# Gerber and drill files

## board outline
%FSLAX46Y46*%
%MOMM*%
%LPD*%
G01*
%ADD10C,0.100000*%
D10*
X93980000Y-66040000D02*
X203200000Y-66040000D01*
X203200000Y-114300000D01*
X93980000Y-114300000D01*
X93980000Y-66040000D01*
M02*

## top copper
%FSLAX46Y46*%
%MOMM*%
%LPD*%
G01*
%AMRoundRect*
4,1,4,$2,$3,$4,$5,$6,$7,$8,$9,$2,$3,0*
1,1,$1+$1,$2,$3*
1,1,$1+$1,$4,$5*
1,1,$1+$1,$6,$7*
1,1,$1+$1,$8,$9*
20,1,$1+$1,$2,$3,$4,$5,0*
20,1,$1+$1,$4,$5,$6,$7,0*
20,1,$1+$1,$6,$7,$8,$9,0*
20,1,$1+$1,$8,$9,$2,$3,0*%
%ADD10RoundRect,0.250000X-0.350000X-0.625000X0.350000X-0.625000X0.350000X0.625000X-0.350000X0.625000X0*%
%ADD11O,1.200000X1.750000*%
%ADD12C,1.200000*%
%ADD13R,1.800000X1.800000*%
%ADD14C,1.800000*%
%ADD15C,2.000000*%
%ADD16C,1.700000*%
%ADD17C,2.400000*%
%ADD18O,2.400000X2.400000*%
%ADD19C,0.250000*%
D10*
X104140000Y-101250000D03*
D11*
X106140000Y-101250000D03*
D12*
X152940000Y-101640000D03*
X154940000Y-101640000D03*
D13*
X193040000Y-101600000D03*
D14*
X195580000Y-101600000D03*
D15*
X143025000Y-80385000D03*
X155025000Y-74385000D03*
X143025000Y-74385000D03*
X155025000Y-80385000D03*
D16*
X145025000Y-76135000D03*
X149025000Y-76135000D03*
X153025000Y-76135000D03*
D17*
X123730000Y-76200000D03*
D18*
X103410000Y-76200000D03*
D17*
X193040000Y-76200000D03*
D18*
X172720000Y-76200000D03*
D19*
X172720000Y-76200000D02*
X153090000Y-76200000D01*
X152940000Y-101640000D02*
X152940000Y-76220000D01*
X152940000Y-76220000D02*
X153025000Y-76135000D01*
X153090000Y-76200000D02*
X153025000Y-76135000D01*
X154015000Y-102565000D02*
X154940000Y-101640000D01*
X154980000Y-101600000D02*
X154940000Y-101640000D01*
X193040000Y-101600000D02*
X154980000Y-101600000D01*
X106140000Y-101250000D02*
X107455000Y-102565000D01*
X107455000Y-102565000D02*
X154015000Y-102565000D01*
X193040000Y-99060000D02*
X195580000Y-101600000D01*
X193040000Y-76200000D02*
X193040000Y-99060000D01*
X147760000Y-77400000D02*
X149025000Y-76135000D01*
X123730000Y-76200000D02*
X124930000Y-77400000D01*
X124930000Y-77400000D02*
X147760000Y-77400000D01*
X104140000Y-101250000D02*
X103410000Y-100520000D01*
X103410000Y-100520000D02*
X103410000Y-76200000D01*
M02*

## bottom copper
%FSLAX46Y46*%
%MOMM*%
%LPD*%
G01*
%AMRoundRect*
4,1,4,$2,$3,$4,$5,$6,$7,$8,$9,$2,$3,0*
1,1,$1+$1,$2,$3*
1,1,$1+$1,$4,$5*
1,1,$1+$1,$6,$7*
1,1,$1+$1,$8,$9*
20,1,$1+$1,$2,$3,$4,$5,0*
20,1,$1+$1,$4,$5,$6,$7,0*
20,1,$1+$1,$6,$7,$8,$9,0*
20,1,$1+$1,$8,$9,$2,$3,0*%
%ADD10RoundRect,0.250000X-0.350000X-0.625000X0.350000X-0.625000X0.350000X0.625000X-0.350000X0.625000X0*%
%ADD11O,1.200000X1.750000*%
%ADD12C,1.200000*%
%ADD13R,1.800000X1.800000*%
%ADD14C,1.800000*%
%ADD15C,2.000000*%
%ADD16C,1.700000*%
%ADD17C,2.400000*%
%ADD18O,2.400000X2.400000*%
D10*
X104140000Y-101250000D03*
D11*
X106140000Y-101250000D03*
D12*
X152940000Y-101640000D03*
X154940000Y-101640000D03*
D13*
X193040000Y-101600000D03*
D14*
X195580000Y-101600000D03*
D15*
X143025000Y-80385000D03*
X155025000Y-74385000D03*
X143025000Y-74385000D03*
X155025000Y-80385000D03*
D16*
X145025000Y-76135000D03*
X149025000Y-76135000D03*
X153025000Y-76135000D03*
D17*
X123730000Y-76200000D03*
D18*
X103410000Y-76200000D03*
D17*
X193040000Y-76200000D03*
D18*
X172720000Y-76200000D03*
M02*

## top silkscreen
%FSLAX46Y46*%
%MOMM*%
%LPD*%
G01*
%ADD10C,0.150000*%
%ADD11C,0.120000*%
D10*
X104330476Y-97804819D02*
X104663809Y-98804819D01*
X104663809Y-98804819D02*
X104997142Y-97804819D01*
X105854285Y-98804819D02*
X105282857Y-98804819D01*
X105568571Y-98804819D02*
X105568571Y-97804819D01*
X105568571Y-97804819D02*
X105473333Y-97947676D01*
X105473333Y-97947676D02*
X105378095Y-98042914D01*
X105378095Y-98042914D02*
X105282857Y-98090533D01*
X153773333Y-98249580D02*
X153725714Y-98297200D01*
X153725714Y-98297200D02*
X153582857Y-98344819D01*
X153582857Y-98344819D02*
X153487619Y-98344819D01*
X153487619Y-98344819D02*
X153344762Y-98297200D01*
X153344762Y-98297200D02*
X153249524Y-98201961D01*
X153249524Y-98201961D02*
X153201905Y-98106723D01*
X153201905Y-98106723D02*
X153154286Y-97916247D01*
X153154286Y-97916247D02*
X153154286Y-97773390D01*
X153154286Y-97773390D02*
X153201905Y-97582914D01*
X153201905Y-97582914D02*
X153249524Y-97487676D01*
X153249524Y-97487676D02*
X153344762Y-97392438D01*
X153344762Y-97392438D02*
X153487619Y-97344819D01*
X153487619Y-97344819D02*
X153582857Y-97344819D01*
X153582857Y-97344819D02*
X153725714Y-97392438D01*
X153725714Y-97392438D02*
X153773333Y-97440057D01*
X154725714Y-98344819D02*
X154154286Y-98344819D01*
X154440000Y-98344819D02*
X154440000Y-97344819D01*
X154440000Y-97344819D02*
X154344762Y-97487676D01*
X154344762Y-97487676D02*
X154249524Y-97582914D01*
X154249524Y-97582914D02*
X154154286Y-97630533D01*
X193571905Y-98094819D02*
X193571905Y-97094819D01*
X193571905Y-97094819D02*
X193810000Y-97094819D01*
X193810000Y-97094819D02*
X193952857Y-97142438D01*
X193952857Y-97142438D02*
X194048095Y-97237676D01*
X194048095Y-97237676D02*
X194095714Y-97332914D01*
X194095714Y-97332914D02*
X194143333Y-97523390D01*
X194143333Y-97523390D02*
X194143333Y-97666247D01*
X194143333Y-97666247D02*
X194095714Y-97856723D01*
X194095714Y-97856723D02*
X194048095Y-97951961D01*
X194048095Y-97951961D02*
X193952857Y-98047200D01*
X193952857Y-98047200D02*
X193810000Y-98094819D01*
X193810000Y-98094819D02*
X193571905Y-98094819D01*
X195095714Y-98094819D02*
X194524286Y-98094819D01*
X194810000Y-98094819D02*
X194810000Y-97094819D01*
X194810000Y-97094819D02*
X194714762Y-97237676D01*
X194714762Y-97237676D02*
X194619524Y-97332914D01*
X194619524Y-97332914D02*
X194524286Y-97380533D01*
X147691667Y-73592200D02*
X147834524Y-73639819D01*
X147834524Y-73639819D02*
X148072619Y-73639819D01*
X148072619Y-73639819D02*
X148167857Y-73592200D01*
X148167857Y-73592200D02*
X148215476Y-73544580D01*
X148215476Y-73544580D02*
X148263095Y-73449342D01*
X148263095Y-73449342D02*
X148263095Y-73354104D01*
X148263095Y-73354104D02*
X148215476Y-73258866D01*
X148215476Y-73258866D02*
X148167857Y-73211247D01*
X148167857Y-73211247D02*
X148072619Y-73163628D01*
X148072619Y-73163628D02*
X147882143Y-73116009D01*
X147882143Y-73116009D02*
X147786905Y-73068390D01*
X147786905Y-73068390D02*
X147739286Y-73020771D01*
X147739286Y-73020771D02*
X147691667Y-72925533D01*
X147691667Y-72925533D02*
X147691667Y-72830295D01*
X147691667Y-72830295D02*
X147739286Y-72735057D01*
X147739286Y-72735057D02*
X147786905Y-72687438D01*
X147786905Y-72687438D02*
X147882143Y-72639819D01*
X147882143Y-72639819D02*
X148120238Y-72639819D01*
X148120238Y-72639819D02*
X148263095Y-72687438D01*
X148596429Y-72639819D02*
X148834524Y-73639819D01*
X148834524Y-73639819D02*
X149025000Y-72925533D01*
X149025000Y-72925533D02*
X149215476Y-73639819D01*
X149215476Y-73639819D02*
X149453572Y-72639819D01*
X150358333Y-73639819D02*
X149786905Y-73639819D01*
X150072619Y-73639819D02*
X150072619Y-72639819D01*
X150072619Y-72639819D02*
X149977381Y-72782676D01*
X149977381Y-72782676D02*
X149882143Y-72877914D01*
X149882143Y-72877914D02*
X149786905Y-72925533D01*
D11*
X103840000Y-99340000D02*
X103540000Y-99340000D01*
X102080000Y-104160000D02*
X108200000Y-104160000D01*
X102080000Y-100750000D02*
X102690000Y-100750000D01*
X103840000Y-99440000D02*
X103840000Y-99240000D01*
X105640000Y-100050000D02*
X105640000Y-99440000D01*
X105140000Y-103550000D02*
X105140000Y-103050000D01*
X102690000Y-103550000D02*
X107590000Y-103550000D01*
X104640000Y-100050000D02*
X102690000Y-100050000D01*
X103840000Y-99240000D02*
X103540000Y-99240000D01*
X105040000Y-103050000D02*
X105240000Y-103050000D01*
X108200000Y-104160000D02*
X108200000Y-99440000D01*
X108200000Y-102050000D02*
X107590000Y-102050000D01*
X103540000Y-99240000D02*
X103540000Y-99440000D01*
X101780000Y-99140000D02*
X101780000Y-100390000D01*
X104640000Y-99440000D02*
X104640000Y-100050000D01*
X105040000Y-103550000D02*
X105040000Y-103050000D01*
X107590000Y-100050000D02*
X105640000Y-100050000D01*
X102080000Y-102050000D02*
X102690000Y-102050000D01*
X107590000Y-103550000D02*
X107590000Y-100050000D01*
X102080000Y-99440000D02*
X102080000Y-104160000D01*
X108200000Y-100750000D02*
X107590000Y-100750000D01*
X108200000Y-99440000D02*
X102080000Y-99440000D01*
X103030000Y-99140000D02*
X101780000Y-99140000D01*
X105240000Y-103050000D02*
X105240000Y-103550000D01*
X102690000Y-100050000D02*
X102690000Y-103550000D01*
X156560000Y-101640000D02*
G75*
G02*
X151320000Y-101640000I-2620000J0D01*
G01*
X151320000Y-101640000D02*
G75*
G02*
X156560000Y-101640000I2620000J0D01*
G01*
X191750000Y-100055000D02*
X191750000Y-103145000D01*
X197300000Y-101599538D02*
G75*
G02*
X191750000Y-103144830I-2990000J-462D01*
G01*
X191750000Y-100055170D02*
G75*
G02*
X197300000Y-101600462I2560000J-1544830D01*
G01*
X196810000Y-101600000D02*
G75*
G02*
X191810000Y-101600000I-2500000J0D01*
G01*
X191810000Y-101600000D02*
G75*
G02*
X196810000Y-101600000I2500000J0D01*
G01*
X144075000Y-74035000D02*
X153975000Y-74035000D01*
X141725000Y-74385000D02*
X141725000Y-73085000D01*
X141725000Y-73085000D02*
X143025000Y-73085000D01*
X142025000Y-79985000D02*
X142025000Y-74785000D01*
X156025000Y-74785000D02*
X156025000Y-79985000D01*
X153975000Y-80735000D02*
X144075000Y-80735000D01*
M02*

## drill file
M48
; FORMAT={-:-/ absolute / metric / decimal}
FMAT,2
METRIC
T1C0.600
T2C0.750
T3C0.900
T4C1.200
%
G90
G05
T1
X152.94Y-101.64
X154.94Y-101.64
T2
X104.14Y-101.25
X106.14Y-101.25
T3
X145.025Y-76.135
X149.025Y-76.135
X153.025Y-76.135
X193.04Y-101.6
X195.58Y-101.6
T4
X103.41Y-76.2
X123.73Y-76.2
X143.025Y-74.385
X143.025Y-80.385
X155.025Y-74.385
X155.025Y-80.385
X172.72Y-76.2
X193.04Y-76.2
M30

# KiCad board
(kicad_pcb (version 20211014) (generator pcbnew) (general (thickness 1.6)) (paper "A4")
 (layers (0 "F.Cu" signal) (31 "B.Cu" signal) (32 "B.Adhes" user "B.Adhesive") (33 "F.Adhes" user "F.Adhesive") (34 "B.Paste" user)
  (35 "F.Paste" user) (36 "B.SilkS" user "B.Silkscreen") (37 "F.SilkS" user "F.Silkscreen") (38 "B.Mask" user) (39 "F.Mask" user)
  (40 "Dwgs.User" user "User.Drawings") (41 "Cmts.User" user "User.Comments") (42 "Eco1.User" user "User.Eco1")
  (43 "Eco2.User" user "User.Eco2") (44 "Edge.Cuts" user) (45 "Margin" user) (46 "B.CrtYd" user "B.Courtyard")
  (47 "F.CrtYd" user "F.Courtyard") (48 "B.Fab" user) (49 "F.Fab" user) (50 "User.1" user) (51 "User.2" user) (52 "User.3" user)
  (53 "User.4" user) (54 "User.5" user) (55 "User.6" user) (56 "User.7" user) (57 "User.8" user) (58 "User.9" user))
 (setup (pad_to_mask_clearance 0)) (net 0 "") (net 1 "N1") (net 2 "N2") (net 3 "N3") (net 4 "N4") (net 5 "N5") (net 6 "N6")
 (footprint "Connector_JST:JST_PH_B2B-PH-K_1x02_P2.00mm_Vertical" (layer "F.Cu") (at 104.14 101.25)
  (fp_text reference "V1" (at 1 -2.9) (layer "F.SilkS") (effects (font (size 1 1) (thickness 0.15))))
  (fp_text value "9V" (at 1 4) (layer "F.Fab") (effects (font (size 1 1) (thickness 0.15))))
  (fp_line (start -0.3 -1.91) (end -0.6 -1.91) (layer "F.SilkS") (width 0.12))
  (fp_line (start -2.06 2.91) (end 4.06 2.91) (layer "F.SilkS") (width 0.12))
  (fp_line (start -2.06 -0.5) (end -1.45 -0.5) (layer "F.SilkS") (width 0.12))
  (fp_line (start -0.3 -1.81) (end -0.3 -2.01) (layer "F.SilkS") (width 0.12))
  (fp_line (start 1.5 -1.2) (end 1.5 -1.81) (layer "F.SilkS") (width 0.12))
  (fp_line (start 1 2.3) (end 1 1.8) (layer "F.SilkS") (width 0.12))
  (fp_line (start -1.45 2.3) (end 3.45 2.3) (layer "F.SilkS") (width 0.12))
  (fp_line (start 0.5 -1.2) (end -1.45 -1.2) (layer "F.SilkS") (width 0.12))
  (fp_line (start -0.3 -2.01) (end -0.6 -2.01) (layer "F.SilkS") (width 0.12))
  (fp_line (start 0.9 1.8) (end 1.1 1.8) (layer "F.SilkS") (width 0.12))
  (fp_line (start 4.06 2.91) (end 4.06 -1.81) (layer "F.SilkS") (width 0.12))
  (fp_line (start 4.06 0.8) (end 3.45 0.8) (layer "F.SilkS") (width 0.12))
  (fp_line (start -0.6 -2.01) (end -0.6 -1.81) (layer "F.SilkS") (width 0.12))
  (fp_line (start -2.36 -2.11) (end -2.36 -0.86) (layer "F.SilkS") (width 0.12))
  (fp_line (start 0.5 -1.81) (end 0.5 -1.2) (layer "F.SilkS") (width 0.12))
  (fp_line (start 0.9 2.3) (end 0.9 1.8) (layer "F.SilkS") (width 0.12))
  (fp_line (start 3.45 -1.2) (end 1.5 -1.2) (layer "F.SilkS") (width 0.12))
  (fp_line (start -2.06 0.8) (end -1.45 0.8) (layer "F.SilkS") (width 0.12))
  (fp_line (start 3.45 2.3) (end 3.45 -1.2) (layer "F.SilkS") (width 0.12))
  (fp_line (start -2.06 -1.81) (end -2.06 2.91) (layer "F.SilkS") (width 0.12))
  (fp_line (start 4.06 -0.5) (end 3.45 -0.5) (layer "F.SilkS") (width 0.12))
  (fp_line (start 4.06 -1.81) (end -2.06 -1.81) (layer "F.SilkS") (width 0.12))
  (fp_line (start -1.11 -2.11) (end -2.36 -2.11) (layer "F.SilkS") (width 0.12))
  (fp_line (start 1.1 1.8) (end 1.1 2.3) (layer "F.SilkS") (width 0.12))
  (fp_line (start -1.45 -1.2) (end -1.45 2.3) (layer "F.SilkS") (width 0.12))
  (pad "1" thru_hole roundrect (at 0 0) (size 1.2 1.75) (drill 0.75) (layers *.Cu *.Mask) (roundrect_rratio 0.208333) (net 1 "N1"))
  (pad "2" thru_hole oval (at 2 0) (size 1.2 1.75) (drill 0.75) (layers *.Cu *.Mask) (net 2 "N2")))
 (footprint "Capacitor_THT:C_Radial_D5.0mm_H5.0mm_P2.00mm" (layer "F.Cu") (at 152.94 101.64)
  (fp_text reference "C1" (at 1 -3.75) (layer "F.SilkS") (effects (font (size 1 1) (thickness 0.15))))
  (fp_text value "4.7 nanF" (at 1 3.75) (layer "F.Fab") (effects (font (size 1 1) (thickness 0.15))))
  (fp_circle (center 1 0) (end 3.62 0) (layer "F.SilkS") (width 0.12) (fill none))
  (pad "1" thru_hole circle (at 0 0) (size 1.2 1.2) (drill 0.6) (layers *.Cu *.Mask) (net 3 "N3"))
  (pad "2" thru_hole circle (at 2 0) (size 1.2 1.2) (drill 0.6) (layers *.Cu *.Mask) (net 2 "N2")))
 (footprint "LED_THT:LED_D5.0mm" (layer "F.Cu") (at 193.04 101.6)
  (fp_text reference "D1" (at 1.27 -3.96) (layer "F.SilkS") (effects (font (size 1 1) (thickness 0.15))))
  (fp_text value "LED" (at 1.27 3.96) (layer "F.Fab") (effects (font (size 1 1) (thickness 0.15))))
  (fp_line (start -1.29 -1.545) (end -1.29 1.545) (layer "F.SilkS") (width 0.12))
  (fp_arc (start 4.26 -0.000462) (mid 2.072002 2.880433) (end -1.29 1.54483) (layer "F.SilkS") (width 0.12))
  (fp_arc (start -1.29 -1.54483) (mid 2.072002 -2.880433) (end 4.26 0.000462) (layer "F.SilkS") (width 0.12))
  (fp_circle (center 1.27 0) (end 3.77 0) (layer "F.SilkS") (width 0.12) (fill none))
  (pad "1" thru_hole rect (at 0 0) (size 1.8 1.8) (drill 0.9) (layers *.Cu *.Mask) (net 2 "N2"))
  (pad "2" thru_hole circle (at 2.54 0) (size 1.8 1.8) (drill 0.9) (layers *.Cu *.Mask) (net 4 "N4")))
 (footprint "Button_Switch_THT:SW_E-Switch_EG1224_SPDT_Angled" (layer "F.Cu") (at 145.025 76.135)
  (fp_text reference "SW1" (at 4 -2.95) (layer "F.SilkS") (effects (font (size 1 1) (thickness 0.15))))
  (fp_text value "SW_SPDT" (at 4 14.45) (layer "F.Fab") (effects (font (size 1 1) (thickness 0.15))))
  (fp_line (start -0.95 -2.1) (end 8.95 -2.1) (layer "F.SilkS") (width 0.12))
  (fp_line (start -3.3 -1.75) (end -3.3 -3.05) (layer "F.SilkS") (width 0.12))
  (fp_line (start -3.3 -3.05) (end -2 -3.05) (layer "F.SilkS") (width 0.12))
  (fp_line (start -3 3.85) (end -3 -1.35) (layer "F.SilkS") (width 0.12))
  (fp_line (start 11 -1.35) (end 11 3.85) (layer "F.SilkS") (width 0.12))
  (fp_line (start 8.95 4.6) (end -0.95 4.6) (layer "F.SilkS") (width 0.12))
  (pad "" thru_hole circle (at -2 4.25) (size 2 2) (drill 1.2) (layers *.Cu *.Mask))
  (pad "" thru_hole circle (at 10 -1.75) (size 2 2) (drill 1.2) (layers *.Cu *.Mask))
  (pad "" thru_hole circle (at -2 -1.75) (size 2 2) (drill 1.2) (layers *.Cu *.Mask))
  (pad "" thru_hole circle (at 10 4.25) (size 2 2) (drill 1.2) (layers *.Cu *.Mask))
  (pad "1" thru_hole circle (at 0 0) (size 1.7 1.7) (drill 0.9) (layers *.Cu *.Mask) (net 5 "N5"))
  (pad "2" thru_hole circle (at 4 0) (size 1.7 1.7) (drill 0.9) (layers *.Cu *.Mask) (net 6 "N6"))
  (pad "3" thru_hole circle (at 8 0) (size 1.7 1.7) (drill 0.9) (layers *.Cu *.Mask) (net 3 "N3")))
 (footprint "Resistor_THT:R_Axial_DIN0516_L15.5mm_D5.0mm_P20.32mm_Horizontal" (layer "B.Cu") (at 123.73 76.2 180)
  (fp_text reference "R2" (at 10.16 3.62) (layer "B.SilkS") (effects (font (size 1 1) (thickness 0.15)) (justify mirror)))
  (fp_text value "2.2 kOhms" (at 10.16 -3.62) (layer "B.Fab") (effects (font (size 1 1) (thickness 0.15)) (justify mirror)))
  (pad "1" thru_hole circle (at 0 0 180) (size 2.4 2.4) (drill 1.2) (layers *.Cu *.Mask) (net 6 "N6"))
  (pad "2" thru_hole oval (at 20.32 0 180) (size 2.4 2.4) (drill 1.2) (layers *.Cu *.Mask) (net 1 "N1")))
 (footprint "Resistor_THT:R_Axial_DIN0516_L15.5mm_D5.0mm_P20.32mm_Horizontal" (layer "B.Cu") (at 193.04 76.2 180)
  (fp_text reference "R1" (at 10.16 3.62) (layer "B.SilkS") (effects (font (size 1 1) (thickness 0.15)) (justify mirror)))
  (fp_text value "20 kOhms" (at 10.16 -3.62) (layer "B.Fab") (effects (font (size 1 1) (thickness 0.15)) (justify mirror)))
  (pad "1" thru_hole circle (at 0 0 180) (size 2.4 2.4) (drill 1.2) (layers *.Cu *.Mask) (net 4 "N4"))
  (pad "2" thru_hole oval (at 20.32 0 180) (size 2.4 2.4) (drill 1.2) (layers *.Cu *.Mask) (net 3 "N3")))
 (gr_rect (start 203.2 114.3) (end 93.98 66.04) (layer "Edge.Cuts") (width 0.1) (fill none))
 (segment (start 172.72 76.2) (end 153.09 76.2) (width 0.25) (layer "F.Cu") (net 3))
 (segment (start 152.94 101.64) (end 152.94 76.22) (width 0.25) (layer "F.Cu") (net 3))
 (segment (start 152.94 76.22) (end 153.025 76.135) (width 0.25) (layer "F.Cu") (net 3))
 (segment (start 153.09 76.2) (end 153.025 76.135) (width 0.25) (layer "F.Cu") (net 3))
 (segment (start 154.015 102.565) (end 154.94 101.64) (width 0.25) (layer "F.Cu") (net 2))
 (segment (start 154.98 101.6) (end 154.94 101.64) (width 0.25) (layer "F.Cu") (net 2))
 (segment (start 193.04 101.6) (end 154.98 101.6) (width 0.25) (layer "F.Cu") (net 2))
 (segment (start 106.14 101.25) (end 107.455 102.565) (width 0.25) (layer "F.Cu") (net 2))
 (segment (start 107.455 102.565) (end 154.015 102.565) (width 0.25) (layer "F.Cu") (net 2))
 (segment (start 193.04 99.06) (end 195.58 101.6) (width 0.25) (layer "F.Cu") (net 4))
 (segment (start 193.04 76.2) (end 193.04 99.06) (width 0.25) (layer "F.Cu") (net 4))
 (segment (start 147.76 77.4) (end 149.025 76.135) (width 0.25) (layer "F.Cu") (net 6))
 (segment (start 123.73 76.2) (end 124.93 77.4) (width 0.25) (layer "F.Cu") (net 6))
 (segment (start 124.93 77.4) (end 147.76 77.4) (width 0.25) (layer "F.Cu") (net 6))
 (segment (start 104.14 101.25) (end 103.41 100.52) (width 0.25) (layer "F.Cu") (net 1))
 (segment (start 103.41 100.52) (end 103.41 76.2) (width 0.25) (layer "F.Cu") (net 1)))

